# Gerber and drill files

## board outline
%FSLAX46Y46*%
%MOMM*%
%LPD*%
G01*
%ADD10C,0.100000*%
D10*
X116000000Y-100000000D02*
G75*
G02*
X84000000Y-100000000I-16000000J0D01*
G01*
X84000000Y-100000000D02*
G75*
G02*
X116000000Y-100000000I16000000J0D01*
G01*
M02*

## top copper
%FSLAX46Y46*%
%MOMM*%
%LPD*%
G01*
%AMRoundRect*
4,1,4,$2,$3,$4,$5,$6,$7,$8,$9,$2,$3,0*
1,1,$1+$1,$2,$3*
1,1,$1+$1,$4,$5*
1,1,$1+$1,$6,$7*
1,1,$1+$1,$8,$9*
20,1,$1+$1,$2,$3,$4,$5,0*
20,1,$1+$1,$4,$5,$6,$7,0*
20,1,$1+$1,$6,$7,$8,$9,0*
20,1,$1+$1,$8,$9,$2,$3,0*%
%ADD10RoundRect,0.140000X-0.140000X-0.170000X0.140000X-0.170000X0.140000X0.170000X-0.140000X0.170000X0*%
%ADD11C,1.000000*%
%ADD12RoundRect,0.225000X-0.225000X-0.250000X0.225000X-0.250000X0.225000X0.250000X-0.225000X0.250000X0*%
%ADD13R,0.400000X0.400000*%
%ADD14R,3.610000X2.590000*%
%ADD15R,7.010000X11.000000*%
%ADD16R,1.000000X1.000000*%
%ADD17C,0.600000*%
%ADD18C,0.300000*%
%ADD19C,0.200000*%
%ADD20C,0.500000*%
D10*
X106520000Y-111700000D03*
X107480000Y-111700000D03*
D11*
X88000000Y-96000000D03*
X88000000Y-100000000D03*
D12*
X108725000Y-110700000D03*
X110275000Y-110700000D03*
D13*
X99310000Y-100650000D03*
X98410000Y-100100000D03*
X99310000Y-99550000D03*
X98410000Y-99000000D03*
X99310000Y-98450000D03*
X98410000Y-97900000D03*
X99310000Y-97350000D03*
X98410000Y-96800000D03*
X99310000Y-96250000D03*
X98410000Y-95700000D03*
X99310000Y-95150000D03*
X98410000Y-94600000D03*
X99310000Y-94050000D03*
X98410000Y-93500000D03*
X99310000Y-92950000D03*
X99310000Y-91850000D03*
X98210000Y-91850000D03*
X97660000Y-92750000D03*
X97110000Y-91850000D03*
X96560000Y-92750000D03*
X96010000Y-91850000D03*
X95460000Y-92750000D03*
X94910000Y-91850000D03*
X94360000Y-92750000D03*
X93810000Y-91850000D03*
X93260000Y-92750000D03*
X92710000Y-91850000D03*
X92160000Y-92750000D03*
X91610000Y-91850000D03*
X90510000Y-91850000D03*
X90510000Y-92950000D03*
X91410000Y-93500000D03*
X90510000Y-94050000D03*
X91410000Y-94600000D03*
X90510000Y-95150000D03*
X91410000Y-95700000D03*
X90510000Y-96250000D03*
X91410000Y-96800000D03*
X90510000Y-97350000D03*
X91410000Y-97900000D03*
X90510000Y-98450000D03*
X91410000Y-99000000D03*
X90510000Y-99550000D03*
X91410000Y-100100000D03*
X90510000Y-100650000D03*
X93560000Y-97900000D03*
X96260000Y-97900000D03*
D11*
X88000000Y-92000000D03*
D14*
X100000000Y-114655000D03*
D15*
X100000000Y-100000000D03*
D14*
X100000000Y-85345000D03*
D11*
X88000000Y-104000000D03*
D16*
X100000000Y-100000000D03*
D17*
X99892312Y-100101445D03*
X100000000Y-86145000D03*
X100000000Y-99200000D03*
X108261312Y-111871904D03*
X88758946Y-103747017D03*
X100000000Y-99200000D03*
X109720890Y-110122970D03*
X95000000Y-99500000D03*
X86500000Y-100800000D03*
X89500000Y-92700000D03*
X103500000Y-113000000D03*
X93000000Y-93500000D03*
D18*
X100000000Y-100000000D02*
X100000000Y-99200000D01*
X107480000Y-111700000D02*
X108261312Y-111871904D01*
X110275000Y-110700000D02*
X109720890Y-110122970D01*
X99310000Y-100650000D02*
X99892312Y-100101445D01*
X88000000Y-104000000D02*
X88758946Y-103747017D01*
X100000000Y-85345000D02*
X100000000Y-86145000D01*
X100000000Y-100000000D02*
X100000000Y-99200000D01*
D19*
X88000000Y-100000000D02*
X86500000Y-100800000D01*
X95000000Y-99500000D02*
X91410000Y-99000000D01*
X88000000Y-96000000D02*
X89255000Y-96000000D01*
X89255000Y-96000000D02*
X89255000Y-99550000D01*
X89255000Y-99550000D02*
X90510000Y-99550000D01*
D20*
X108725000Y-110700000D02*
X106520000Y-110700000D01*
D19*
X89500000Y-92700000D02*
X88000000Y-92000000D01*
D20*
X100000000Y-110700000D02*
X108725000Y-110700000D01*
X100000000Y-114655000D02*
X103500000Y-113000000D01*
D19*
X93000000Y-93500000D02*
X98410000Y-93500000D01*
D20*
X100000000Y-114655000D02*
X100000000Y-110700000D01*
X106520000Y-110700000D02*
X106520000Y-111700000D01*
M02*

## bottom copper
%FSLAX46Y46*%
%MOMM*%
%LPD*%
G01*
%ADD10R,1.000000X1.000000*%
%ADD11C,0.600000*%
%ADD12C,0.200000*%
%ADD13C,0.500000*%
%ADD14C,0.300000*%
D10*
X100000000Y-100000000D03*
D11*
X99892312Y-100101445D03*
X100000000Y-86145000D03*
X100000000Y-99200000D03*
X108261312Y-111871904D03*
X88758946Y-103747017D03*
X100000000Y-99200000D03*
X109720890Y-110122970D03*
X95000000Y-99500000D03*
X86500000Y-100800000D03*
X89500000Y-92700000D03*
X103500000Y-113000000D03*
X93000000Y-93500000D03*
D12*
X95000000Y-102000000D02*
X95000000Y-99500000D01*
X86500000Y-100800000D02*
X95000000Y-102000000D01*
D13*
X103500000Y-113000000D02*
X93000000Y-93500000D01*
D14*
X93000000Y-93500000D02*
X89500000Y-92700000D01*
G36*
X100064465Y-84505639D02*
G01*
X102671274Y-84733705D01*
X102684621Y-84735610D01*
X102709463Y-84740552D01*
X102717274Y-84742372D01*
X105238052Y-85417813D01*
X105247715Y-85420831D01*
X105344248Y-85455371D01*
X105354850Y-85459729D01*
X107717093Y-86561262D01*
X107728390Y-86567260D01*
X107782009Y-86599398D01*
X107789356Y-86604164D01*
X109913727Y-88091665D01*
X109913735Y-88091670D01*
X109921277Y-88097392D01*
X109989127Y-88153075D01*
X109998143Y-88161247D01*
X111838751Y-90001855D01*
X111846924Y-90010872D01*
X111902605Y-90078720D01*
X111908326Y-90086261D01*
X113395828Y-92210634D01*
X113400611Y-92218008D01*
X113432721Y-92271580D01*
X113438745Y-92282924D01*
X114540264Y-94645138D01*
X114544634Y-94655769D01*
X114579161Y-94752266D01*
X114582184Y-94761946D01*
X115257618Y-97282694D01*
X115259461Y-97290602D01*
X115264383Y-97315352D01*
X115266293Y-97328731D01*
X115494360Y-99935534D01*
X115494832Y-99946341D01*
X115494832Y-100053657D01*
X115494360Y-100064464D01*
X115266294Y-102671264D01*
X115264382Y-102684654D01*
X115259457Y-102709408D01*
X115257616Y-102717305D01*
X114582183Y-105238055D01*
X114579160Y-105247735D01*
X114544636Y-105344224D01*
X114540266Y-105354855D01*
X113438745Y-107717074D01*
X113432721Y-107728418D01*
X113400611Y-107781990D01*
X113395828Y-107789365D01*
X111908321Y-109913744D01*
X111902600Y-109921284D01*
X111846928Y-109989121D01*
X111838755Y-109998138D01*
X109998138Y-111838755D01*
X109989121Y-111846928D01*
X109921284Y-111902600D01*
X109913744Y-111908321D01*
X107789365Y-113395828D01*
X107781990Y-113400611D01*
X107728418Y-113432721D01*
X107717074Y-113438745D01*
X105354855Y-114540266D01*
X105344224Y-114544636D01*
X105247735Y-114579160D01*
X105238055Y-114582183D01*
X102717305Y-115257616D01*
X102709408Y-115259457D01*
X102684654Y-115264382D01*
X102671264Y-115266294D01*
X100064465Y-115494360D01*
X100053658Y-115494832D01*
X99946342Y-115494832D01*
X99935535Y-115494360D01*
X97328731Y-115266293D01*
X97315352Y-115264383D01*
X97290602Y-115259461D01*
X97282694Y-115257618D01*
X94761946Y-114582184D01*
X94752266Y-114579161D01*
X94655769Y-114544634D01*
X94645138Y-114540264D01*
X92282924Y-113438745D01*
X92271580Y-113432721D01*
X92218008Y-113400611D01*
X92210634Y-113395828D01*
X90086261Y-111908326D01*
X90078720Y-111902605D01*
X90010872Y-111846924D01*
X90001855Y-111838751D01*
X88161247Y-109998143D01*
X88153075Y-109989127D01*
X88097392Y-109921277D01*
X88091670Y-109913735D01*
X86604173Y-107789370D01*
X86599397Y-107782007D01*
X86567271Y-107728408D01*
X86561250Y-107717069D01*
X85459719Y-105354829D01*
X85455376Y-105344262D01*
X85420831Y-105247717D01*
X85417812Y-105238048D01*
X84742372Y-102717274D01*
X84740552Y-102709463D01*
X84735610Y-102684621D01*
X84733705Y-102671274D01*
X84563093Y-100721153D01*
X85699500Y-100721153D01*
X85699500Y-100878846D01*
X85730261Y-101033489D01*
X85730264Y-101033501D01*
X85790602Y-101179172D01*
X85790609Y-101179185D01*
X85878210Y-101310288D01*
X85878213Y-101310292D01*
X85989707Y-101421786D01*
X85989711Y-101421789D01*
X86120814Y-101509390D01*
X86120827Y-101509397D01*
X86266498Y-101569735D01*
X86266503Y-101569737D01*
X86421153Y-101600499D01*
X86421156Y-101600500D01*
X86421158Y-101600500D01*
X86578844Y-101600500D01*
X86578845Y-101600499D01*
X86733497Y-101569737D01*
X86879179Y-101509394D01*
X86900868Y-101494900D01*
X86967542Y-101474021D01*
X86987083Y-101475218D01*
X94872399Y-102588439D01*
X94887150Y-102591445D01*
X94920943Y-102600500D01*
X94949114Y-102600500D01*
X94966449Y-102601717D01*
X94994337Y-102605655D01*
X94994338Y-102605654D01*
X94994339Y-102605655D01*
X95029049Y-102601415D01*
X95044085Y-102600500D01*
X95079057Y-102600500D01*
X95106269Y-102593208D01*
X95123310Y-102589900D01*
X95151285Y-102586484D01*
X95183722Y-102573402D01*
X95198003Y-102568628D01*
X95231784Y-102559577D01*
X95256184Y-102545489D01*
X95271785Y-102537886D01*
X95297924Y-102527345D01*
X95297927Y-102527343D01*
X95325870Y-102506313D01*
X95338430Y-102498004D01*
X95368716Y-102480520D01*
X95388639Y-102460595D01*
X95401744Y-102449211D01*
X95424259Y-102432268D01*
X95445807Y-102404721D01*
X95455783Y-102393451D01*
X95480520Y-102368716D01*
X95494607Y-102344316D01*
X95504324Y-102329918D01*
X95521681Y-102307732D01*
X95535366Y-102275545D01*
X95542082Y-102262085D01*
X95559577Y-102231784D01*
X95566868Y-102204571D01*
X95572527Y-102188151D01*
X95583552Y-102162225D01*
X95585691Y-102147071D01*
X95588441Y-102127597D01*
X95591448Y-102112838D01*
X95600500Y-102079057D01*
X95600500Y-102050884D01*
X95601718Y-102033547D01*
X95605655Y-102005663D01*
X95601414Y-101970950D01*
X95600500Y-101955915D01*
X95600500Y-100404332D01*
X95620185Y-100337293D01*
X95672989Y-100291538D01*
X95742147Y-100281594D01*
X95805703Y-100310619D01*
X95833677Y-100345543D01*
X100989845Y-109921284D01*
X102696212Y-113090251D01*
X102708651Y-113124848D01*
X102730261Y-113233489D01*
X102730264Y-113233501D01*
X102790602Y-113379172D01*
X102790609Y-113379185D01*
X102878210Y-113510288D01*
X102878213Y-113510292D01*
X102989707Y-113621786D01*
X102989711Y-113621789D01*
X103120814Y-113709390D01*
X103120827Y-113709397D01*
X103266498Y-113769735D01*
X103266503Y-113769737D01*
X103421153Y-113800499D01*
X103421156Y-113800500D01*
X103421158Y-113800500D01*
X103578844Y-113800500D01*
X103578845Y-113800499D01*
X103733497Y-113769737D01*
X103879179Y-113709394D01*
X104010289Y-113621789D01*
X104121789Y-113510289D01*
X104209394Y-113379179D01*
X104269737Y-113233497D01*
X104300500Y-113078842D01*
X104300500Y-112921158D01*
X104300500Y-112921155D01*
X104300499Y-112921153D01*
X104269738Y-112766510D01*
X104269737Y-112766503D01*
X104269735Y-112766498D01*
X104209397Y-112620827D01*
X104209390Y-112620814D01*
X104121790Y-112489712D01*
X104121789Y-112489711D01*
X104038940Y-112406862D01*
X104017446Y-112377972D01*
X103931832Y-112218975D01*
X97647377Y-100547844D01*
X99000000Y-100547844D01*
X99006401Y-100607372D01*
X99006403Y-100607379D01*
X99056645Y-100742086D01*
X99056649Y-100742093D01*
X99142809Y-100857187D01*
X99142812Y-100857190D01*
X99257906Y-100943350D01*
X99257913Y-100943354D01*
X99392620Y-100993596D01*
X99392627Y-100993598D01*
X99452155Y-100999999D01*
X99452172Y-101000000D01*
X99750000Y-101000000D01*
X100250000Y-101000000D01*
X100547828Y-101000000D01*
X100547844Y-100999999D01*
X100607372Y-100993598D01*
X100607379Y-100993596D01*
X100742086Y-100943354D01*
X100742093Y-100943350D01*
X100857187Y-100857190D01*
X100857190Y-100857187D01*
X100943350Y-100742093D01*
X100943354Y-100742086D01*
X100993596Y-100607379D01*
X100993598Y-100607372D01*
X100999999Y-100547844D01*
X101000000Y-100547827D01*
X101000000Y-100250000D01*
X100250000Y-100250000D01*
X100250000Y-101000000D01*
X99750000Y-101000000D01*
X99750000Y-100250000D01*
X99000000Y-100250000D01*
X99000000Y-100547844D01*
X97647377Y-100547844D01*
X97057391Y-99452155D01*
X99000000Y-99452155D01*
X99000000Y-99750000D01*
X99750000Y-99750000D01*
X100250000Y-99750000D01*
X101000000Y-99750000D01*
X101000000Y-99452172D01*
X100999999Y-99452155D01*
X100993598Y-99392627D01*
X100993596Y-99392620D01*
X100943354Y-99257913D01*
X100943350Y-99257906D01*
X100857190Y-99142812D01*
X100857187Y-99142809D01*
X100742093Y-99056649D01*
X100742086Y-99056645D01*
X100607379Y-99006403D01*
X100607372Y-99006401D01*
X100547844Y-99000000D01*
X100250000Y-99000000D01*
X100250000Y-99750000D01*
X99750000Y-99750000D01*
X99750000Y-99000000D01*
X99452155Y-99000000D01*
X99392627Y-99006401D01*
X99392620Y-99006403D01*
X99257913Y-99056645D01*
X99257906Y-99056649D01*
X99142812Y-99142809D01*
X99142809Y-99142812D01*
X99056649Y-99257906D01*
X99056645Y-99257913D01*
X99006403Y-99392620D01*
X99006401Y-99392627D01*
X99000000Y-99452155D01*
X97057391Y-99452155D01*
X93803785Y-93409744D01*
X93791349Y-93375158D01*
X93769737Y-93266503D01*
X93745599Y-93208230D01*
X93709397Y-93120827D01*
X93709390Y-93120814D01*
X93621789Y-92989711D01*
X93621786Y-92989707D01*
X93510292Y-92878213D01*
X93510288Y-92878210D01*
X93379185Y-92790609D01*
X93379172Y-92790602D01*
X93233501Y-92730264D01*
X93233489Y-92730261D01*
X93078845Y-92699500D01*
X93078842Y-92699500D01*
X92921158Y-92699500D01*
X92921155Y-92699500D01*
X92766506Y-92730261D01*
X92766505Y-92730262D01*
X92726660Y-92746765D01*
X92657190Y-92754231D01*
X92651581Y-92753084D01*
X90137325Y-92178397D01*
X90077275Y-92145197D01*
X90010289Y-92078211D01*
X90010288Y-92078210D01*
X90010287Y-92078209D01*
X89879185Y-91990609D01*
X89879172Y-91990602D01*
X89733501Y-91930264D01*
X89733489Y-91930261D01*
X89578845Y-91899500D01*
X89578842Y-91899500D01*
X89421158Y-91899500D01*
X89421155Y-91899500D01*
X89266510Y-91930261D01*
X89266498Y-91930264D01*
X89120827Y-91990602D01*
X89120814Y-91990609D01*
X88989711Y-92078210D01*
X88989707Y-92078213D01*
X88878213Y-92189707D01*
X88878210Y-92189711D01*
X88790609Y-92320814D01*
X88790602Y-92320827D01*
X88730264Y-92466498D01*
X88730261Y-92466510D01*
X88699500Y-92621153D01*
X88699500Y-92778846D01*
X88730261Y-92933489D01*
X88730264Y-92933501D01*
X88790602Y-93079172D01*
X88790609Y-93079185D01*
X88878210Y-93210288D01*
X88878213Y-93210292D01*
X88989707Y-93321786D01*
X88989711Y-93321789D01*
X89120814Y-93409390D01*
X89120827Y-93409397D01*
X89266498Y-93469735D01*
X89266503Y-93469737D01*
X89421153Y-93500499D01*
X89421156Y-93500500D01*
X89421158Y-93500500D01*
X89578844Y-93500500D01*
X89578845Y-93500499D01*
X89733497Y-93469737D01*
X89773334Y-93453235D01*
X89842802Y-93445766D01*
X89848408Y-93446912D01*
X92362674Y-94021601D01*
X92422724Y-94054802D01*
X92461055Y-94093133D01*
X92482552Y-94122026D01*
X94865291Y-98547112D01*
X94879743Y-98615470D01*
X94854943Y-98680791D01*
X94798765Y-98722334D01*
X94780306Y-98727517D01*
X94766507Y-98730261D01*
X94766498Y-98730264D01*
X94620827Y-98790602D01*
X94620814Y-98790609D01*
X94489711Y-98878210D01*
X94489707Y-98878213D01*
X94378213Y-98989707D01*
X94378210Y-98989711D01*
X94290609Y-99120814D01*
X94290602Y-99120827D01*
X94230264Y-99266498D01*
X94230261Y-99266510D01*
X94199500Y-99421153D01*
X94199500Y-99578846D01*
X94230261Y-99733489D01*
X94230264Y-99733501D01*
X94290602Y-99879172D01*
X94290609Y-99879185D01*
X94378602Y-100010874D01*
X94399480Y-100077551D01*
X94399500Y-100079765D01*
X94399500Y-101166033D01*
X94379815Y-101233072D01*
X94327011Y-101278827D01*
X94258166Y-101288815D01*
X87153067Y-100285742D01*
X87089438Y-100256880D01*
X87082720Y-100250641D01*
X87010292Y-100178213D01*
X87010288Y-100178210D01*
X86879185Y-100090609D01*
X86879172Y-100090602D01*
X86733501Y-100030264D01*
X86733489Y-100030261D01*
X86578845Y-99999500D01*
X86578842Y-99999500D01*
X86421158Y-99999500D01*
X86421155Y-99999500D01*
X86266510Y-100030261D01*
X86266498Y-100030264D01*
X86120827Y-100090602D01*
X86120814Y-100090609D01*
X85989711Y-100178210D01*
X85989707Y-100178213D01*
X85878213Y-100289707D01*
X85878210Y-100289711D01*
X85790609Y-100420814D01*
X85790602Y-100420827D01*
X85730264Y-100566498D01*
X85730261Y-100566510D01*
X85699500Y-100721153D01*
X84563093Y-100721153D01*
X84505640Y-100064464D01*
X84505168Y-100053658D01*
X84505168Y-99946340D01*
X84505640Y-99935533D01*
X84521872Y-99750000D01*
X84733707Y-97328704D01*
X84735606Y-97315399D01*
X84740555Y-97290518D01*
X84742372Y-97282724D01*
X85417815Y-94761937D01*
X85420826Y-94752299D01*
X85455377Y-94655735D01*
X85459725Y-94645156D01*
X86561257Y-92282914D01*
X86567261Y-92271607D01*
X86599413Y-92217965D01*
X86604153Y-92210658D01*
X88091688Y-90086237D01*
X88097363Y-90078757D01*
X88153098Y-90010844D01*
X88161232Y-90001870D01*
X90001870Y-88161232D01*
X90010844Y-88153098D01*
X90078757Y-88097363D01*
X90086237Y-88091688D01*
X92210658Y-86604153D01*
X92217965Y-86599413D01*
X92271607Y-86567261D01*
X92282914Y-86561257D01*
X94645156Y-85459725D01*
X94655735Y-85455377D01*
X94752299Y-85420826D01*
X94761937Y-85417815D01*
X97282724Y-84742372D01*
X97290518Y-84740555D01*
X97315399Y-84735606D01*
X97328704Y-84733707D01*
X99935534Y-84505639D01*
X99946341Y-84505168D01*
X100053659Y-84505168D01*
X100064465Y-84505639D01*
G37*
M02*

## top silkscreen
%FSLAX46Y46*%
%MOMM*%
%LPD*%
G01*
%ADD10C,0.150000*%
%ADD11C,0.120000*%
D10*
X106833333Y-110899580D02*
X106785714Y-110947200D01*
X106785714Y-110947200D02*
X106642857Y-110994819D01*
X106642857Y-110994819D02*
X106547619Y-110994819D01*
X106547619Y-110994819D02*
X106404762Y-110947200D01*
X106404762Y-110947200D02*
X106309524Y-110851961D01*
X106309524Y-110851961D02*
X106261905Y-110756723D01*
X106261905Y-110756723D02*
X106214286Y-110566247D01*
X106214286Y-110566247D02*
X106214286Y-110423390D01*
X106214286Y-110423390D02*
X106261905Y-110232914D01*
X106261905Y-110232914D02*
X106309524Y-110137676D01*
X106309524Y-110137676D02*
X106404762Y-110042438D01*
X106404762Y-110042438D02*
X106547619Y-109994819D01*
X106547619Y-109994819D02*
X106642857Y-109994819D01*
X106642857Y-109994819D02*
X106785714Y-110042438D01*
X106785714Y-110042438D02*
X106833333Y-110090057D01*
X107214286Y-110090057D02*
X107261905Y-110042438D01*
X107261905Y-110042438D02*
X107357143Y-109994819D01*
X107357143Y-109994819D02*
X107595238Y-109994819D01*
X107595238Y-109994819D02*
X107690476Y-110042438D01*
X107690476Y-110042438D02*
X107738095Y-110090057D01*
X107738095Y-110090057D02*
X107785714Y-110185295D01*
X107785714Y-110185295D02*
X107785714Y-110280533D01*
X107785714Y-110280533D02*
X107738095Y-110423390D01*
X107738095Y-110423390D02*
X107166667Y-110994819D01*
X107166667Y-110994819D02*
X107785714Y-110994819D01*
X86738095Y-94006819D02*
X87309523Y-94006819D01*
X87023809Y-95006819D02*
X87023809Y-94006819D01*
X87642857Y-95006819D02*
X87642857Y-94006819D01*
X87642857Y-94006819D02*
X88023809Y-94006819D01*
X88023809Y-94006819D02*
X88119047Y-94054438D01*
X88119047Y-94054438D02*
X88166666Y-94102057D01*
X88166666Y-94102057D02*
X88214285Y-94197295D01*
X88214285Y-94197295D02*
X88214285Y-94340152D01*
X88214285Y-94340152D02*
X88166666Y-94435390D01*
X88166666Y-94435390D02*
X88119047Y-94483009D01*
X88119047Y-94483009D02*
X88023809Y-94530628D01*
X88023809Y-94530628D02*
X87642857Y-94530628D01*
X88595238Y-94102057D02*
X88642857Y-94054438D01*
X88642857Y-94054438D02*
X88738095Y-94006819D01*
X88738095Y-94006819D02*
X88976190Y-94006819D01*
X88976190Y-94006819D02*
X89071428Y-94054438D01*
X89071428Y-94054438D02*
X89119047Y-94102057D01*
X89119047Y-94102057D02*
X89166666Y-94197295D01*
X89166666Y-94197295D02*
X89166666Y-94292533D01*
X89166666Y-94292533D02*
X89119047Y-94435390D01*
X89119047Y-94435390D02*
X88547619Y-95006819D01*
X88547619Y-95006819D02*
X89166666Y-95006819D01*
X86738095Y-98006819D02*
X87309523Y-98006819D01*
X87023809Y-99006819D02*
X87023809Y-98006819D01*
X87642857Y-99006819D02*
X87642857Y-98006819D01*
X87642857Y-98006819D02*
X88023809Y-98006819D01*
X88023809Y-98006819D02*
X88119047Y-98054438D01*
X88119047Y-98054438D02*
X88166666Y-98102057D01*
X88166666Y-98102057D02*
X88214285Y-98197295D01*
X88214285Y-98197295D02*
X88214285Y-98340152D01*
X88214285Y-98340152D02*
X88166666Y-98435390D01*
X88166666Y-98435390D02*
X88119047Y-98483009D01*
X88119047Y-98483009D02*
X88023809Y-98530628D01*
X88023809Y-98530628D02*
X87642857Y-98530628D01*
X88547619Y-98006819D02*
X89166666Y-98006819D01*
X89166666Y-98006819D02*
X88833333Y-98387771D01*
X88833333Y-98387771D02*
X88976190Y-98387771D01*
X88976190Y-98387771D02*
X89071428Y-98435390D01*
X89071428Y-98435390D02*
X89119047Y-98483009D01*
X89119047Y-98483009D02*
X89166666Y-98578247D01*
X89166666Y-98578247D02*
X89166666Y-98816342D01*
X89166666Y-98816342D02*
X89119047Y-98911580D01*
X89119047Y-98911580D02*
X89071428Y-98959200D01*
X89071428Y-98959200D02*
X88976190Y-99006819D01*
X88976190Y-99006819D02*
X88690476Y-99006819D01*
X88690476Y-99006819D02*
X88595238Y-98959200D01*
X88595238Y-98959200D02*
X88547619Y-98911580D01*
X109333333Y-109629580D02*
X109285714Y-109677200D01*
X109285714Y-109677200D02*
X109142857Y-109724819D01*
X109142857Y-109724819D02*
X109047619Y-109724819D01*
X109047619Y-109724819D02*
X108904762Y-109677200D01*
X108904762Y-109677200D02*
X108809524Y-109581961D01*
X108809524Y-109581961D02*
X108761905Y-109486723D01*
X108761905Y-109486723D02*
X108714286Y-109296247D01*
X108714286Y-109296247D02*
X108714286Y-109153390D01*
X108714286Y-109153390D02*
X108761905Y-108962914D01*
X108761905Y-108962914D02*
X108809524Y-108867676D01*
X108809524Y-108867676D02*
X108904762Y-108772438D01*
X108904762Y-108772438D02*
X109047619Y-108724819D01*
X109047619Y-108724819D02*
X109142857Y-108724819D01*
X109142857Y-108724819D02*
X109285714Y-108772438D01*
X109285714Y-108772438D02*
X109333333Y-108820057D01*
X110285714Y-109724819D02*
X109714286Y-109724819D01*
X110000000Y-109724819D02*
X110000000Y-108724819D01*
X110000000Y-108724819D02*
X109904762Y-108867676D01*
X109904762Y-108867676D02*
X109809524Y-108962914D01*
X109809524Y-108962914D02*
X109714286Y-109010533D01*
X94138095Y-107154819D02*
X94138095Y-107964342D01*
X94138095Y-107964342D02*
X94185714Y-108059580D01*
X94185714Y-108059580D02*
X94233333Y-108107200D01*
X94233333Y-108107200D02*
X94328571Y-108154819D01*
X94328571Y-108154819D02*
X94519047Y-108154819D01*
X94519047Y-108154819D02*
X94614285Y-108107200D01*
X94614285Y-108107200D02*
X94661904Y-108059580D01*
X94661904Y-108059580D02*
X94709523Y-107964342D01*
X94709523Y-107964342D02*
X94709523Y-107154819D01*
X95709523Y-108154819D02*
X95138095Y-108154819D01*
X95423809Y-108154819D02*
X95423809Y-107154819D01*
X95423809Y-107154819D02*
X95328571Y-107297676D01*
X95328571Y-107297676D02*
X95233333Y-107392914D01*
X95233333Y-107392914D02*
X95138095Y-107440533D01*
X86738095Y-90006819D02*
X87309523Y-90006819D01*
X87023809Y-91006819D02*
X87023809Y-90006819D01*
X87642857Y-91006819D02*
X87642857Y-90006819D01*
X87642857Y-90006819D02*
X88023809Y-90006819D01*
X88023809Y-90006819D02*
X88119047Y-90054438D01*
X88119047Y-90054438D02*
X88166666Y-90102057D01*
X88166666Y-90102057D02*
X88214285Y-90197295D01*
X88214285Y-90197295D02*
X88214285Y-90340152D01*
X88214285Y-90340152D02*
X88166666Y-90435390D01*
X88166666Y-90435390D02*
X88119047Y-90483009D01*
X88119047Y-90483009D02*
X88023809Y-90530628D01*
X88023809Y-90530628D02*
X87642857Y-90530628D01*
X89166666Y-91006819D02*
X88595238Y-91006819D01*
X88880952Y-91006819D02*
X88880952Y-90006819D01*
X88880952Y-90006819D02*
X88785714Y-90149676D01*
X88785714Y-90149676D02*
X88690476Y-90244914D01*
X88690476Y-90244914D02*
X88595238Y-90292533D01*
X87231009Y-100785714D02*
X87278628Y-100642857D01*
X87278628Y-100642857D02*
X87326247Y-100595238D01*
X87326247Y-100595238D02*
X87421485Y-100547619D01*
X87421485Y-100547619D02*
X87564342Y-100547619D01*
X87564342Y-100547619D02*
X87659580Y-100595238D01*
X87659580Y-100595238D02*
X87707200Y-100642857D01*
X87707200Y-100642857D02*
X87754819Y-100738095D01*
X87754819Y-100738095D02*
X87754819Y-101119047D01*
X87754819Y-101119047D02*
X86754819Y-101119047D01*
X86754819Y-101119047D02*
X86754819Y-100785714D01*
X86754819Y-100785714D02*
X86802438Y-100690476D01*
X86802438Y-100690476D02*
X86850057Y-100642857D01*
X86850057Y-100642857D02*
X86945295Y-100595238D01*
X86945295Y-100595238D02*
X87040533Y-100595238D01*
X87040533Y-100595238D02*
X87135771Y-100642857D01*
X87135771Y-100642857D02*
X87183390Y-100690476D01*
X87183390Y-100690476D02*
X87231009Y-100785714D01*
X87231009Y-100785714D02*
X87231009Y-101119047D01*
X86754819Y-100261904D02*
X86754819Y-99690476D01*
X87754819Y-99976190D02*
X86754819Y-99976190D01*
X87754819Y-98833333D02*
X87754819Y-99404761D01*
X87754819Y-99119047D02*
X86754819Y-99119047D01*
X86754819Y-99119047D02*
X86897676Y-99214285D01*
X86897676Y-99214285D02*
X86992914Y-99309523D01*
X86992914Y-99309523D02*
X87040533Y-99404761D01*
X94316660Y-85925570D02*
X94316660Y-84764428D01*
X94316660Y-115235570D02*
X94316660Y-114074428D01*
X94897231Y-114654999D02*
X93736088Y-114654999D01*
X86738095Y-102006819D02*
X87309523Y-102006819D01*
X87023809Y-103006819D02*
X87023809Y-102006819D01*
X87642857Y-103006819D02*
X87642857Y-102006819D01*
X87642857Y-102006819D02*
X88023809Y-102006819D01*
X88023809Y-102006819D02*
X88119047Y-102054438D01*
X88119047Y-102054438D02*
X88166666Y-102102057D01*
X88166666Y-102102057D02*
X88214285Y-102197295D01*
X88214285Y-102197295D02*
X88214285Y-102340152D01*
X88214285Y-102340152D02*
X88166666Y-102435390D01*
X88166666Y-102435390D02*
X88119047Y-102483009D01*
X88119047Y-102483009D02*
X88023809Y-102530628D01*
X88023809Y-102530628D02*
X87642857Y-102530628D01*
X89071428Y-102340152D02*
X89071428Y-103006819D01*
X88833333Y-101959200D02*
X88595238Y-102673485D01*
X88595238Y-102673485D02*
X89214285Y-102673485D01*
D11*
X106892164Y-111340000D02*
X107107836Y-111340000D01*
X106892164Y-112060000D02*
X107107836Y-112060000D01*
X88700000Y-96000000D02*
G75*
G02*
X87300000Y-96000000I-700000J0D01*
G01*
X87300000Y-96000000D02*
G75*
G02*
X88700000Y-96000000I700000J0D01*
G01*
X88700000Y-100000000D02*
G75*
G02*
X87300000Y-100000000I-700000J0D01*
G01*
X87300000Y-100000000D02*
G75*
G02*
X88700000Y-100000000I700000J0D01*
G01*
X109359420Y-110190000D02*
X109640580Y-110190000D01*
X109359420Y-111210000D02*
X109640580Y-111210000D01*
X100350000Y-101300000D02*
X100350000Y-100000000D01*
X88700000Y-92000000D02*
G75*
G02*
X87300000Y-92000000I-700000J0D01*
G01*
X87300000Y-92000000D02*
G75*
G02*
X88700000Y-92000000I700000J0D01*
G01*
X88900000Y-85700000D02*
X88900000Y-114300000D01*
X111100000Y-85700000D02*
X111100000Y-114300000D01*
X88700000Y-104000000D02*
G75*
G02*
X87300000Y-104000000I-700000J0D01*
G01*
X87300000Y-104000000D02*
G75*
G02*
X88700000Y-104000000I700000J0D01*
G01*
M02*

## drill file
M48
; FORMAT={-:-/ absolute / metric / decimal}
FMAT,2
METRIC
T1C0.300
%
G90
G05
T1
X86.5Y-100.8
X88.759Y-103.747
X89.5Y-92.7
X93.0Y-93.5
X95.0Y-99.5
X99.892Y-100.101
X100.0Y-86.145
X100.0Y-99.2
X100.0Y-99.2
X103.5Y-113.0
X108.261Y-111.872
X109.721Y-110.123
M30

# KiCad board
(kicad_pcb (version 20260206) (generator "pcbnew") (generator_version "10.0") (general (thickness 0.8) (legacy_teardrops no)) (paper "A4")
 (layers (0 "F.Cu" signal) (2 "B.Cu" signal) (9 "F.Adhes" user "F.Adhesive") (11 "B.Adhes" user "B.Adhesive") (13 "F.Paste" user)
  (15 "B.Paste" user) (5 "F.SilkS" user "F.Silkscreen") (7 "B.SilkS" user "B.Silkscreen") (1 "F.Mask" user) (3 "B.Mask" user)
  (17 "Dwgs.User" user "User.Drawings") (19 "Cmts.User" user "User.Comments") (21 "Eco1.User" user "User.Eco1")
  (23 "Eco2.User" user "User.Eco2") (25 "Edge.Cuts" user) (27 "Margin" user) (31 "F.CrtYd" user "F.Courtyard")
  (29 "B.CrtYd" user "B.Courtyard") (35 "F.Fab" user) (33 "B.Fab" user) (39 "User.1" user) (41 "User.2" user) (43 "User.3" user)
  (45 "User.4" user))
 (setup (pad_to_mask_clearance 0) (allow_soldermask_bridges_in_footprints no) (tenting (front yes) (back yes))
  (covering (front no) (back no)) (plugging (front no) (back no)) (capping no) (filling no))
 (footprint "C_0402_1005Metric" (layer "F.Cu") (at 107 111.7)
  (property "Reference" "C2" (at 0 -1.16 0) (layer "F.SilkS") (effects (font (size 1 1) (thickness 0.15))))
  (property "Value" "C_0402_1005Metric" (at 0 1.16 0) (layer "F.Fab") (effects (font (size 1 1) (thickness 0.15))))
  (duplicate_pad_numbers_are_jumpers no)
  (fp_line (start -0.107836 -0.36) (end 0.107836 -0.36) (stroke (width 0.12) (type solid)) (layer "F.SilkS"))
  (fp_line (start -0.107836 0.36) (end 0.107836 0.36) (stroke (width 0.12) (type solid)) (layer "F.SilkS"))
  (pad "1" smd roundrect (at -0.48 0) (size 0.56 0.62) (layers "F.Cu" "F.Mask" "F.Paste") (roundrect_rratio 0.25) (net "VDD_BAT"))
  (pad "2" smd roundrect (at 0.48 0) (size 0.56 0.62) (layers "F.Cu" "F.Mask" "F.Paste") (roundrect_rratio 0.25) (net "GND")))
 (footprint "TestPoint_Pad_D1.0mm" (layer "F.Cu") (at 88 96)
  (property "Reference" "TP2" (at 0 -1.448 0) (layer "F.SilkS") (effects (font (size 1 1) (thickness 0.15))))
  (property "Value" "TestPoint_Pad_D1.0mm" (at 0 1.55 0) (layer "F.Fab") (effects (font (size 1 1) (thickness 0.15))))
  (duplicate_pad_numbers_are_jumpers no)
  (fp_circle (center 0 0) (end 0 0.7) (stroke (width 0.12) (type solid)) (fill no) (layer "F.SilkS"))
  (pad "1" smd circle (at 0 0) (size 1 1) (layers "F.Cu" "F.Mask") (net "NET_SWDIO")))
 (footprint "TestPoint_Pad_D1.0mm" (layer "F.Cu") (at 88 100)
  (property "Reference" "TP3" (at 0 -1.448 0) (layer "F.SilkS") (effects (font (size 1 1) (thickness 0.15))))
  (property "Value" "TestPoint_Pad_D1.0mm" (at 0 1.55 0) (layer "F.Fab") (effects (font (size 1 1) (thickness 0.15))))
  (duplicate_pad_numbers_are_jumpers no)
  (fp_circle (center 0 0) (end 0 0.7) (stroke (width 0.12) (type solid)) (fill no) (layer "F.SilkS"))
  (pad "1" smd circle (at 0 0) (size 1 1) (layers "F.Cu" "F.Mask") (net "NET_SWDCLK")))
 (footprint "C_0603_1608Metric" (layer "F.Cu") (at 109.5 110.7)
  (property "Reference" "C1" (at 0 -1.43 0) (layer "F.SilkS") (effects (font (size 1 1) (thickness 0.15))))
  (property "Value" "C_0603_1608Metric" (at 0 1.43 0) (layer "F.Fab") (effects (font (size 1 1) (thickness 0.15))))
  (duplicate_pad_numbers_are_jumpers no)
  (fp_line (start -0.14058 -0.51) (end 0.14058 -0.51) (stroke (width 0.12) (type solid)) (layer "F.SilkS"))
  (fp_line (start -0.14058 0.51) (end 0.14058 0.51) (stroke (width 0.12) (type solid)) (layer "F.SilkS"))
  (pad "1" smd roundrect (at -0.775 0) (size 0.9 0.95) (layers "F.Cu" "F.Mask" "F.Paste") (roundrect_rratio 0.25) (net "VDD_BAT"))
  (pad "2" smd roundrect (at 0.775 0) (size 0.9 0.95) (layers "F.Cu" "F.Mask" "F.Paste") (roundrect_rratio 0.25) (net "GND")))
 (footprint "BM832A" (layer "F.Cu") (at 100 106.2 180)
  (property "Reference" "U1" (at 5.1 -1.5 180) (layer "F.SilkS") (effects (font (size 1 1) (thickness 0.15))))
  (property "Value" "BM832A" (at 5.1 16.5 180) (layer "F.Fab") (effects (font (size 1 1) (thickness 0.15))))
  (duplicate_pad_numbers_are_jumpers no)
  (fp_line (start -0.35 4.9) (end -0.35 6.2) (stroke (width 0.12) (type solid)) (layer "F.SilkS"))
  (pad "1" smd rect (at 0.69 5.55 180) (size 0.4 0.4) (layers "F.Cu" "F.Mask" "F.Paste") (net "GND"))
  (pad "2" smd rect (at 1.59 6.1 180) (size 0.4 0.4) (layers "F.Cu" "F.Mask" "F.Paste"))
  (pad "3" smd rect (at 0.69 6.65 180) (size 0.4 0.4) (layers "F.Cu" "F.Mask" "F.Paste"))
  (pad "4" smd rect (at 1.59 7.2 180) (size 0.4 0.4) (layers "F.Cu" "F.Mask" "F.Paste"))
  (pad "5" smd rect (at 0.69 7.75 180) (size 0.4 0.4) (layers "F.Cu" "F.Mask" "F.Paste"))
  (pad "6" smd rect (at 1.59 8.3 180) (size 0.4 0.4) (layers "F.Cu" "F.Mask" "F.Paste"))
  (pad "7" smd rect (at 0.69 8.85 180) (size 0.4 0.4) (layers "F.Cu" "F.Mask" "F.Paste"))
  (pad "8" smd rect (at 1.59 9.4 180) (size 0.4 0.4) (layers "F.Cu" "F.Mask" "F.Paste"))
  (pad "9" smd rect (at 0.69 9.95 180) (size 0.4 0.4) (layers "F.Cu" "F.Mask" "F.Paste"))
  (pad "10" smd rect (at 1.59 10.5 180) (size 0.4 0.4) (layers "F.Cu" "F.Mask" "F.Paste"))
  (pad "11" smd rect (at 0.69 11.05 180) (size 0.4 0.4) (layers "F.Cu" "F.Mask" "F.Paste"))
  (pad "12" smd rect (at 1.59 11.6 180) (size 0.4 0.4) (layers "F.Cu" "F.Mask" "F.Paste"))
  (pad "13" smd rect (at 0.69 12.15 180) (size 0.4 0.4) (layers "F.Cu" "F.Mask" "F.Paste"))
  (pad "14" smd rect (at 1.59 12.7 180) (size 0.4 0.4) (layers "F.Cu" "F.Mask" "F.Paste") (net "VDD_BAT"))
  (pad "15" smd rect (at 0.69 13.25 180) (size 0.4 0.4) (layers "F.Cu" "F.Mask" "F.Paste"))
  (pad "16" smd rect (at 0.69 14.35 180) (size 0.4 0.4) (layers "F.Cu" "F.Mask" "F.Paste"))
  (pad "17" smd rect (at 1.79 14.35 180) (size 0.4 0.4) (layers "F.Cu" "F.Mask" "F.Paste"))
  (pad "18" smd rect (at 2.34 13.45 180) (size 0.4 0.4) (layers "F.Cu" "F.Mask" "F.Paste"))
  (pad "19" smd rect (at 2.89 14.35 180) (size 0.4 0.4) (layers "F.Cu" "F.Mask" "F.Paste"))
  (pad "20" smd rect (at 3.44 13.45 180) (size 0.4 0.4) (layers "F.Cu" "F.Mask" "F.Paste"))
  (pad "21" smd rect (at 3.99 14.35 180) (size 0.4 0.4) (layers "F.Cu" "F.Mask" "F.Paste"))
  (pad "22" smd rect (at 4.54 13.45 180) (size 0.4 0.4) (layers "F.Cu" "F.Mask" "F.Paste"))
  (pad "23" smd rect (at 5.09 14.35 180) (size 0.4 0.4) (layers "F.Cu" "F.Mask" "F.Paste"))
  (pad "24" smd rect (at 5.64 13.45 180) (size 0.4 0.4) (layers "F.Cu" "F.Mask" "F.Paste"))
  (pad "25" smd rect (at 6.19 14.35 180) (size 0.4 0.4) (layers "F.Cu" "F.Mask" "F.Paste"))
  (pad "26" smd rect (at 6.74 13.45 180) (size 0.4 0.4) (layers "F.Cu" "F.Mask" "F.Paste"))
  (pad "27" smd rect (at 7.29 14.35 180) (size 0.4 0.4) (layers "F.Cu" "F.Mask" "F.Paste"))
  (pad "28" smd rect (at 7.84 13.45 180) (size 0.4 0.4) (layers "F.Cu" "F.Mask" "F.Paste"))
  (pad "29" smd rect (at 8.39 14.35 180) (size 0.4 0.4) (layers "F.Cu" "F.Mask" "F.Paste"))
  (pad "30" smd rect (at 9.49 14.35 180) (size 0.4 0.4) (layers "F.Cu" "F.Mask" "F.Paste"))
  (pad "31" smd rect (at 9.49 13.25 180) (size 0.4 0.4) (layers "F.Cu" "F.Mask" "F.Paste"))
  (pad "32" smd rect (at 8.59 12.7 180) (size 0.4 0.4) (layers "F.Cu" "F.Mask" "F.Paste"))
  (pad "33" smd rect (at 9.49 12.15 180) (size 0.4 0.4) (layers "F.Cu" "F.Mask" "F.Paste"))
  (pad "34" smd rect (at 8.59 11.6 180) (size 0.4 0.4) (layers "F.Cu" "F.Mask" "F.Paste"))
  (pad "35" smd rect (at 9.49 11.05 180) (size 0.4 0.4) (layers "F.Cu" "F.Mask" "F.Paste"))
  (pad "36" smd rect (at 8.59 10.5 180) (size 0.4 0.4) (layers "F.Cu" "F.Mask" "F.Paste"))
  (pad "37" smd rect (at 9.49 9.95 180) (size 0.4 0.4) (layers "F.Cu" "F.Mask" "F.Paste"))
  (pad "38" smd rect (at 8.59 9.4 180) (size 0.4 0.4) (layers "F.Cu" "F.Mask" "F.Paste"))
  (pad "39" smd rect (at 9.49 8.85 180) (size 0.4 0.4) (layers "F.Cu" "F.Mask" "F.Paste"))
  (pad "40" smd rect (at 8.59 8.3 180) (size 0.4 0.4) (layers "F.Cu" "F.Mask" "F.Paste"))
  (pad "41" smd rect (at 9.49 7.75 180) (size 0.4 0.4) (layers "F.Cu" "F.Mask" "F.Paste"))
  (pad "42" smd rect (at 8.59 7.2 180) (size 0.4 0.4) (layers "F.Cu" "F.Mask" "F.Paste") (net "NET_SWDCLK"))
  (pad "43" smd rect (at 9.49 6.65 180) (size 0.4 0.4) (layers "F.Cu" "F.Mask" "F.Paste") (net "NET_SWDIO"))
  (pad "44" smd rect (at 8.59 6.1 180) (size 0.4 0.4) (layers "F.Cu" "F.Mask" "F.Paste"))
  (pad "45" smd rect (at 9.49 5.55 180) (size 0.4 0.4) (layers "F.Cu" "F.Mask" "F.Paste"))
  (pad "46" smd rect (at 6.44 8.3 180) (size 0.4 0.4) (layers "F.Cu" "F.Mask" "F.Paste"))
  (pad "47" smd rect (at 3.74 8.3 180) (size 0.4 0.4) (layers "F.Cu" "F.Mask" "F.Paste")))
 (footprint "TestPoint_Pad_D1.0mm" (layer "F.Cu") (at 88 92)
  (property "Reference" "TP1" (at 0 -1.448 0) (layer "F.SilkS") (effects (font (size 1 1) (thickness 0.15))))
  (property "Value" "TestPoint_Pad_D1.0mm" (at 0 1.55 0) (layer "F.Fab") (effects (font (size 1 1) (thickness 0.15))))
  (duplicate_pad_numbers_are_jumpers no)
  (fp_circle (center 0 0) (end 0 0.7) (stroke (width 0.12) (type solid)) (fill no) (layer "F.SilkS"))
  (pad "1" smd circle (at 0 0) (size 1 1) (layers "F.Cu" "F.Mask") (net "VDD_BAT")))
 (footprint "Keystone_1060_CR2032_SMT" (layer "F.Cu") (at 100 100 -90)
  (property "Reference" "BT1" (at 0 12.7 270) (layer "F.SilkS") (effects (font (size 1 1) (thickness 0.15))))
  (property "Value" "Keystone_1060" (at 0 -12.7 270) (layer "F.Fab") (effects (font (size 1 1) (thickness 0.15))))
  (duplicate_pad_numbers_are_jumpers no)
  (fp_line (start -14.3 11.1) (end 14.3 11.1) (stroke (width 0.12) (type solid)) (layer "F.SilkS"))
  (fp_line (start -14.3 -11.1) (end 14.3 -11.1) (stroke (width 0.12) (type solid)) (layer "F.SilkS"))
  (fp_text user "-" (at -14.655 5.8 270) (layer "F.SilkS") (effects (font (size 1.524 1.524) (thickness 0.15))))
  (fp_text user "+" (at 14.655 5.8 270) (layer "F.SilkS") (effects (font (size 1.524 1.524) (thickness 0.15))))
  (pad "1" smd rect (at 14.655 0 270) (size 2.59 3.61) (layers "F.Cu" "F.Mask" "F.Paste") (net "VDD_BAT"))
  (pad "2" smd rect (at 0 0 270) (size 11 7.01) (layers "F.Cu" "F.Mask" "F.Paste") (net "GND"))
  (pad "3" smd rect (at -14.655 0 270) (size 2.59 3.61) (layers "F.Cu" "F.Mask" "F.Paste") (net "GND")))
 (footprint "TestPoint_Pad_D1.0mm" (layer "F.Cu") (at 88 104)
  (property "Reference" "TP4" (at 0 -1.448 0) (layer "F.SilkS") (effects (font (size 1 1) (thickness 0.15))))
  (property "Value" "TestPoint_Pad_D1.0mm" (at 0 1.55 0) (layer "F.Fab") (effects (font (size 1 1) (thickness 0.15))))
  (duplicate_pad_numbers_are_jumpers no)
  (fp_circle (center 0 0) (end 0 0.7) (stroke (width 0.12) (type solid)) (fill no) (layer "F.SilkS"))
  (pad "1" smd circle (at 0 0) (size 1 1) (layers "F.Cu" "F.Mask") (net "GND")))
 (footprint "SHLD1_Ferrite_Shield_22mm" (layer "B.Cu") (at 100 100 180)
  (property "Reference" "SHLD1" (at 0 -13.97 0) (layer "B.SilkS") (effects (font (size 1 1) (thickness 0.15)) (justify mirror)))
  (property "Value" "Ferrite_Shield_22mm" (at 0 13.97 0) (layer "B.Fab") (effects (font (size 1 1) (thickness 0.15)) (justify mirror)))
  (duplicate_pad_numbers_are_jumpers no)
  (pad "1" smd rect (at 0 0 180) (size 1 1) (layers "*.Cu" "*.Paste" "*.Mask") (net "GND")))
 (gr_circle (center 100 100) (end 116 100) (stroke (width 0.1) (type default)) (fill no) (layer "Edge.Cuts"))
 (segment (start 100 100) (end 100 99.2) (width 0.3) (layer "F.Cu") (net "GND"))
 (segment (start 107.48 111.7) (end 108.261312 111.871904) (width 0.3) (layer "F.Cu") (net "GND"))
 (segment (start 110.275 110.7) (end 109.72089 110.12297) (width 0.3) (layer "F.Cu") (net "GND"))
 (segment (start 99.31 100.65) (end 99.892312 100.101445) (width 0.3) (layer "F.Cu") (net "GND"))
 (segment (start 88 104) (end 88.758946 103.747017) (width 0.3) (layer "F.Cu") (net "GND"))
 (segment (start 100 85.345) (end 100 86.145) (width 0.3) (layer "F.Cu") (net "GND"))
 (segment (start 100 100) (end 100 99.2) (width 0.3) (layer "F.Cu") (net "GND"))
 (via (at 99.892312 100.101445) (size 0.6) (drill 0.3) (layers "F.Cu" "B.Cu") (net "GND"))
 (via (at 100 86.145) (size 0.6) (drill 0.3) (layers "F.Cu" "B.Cu") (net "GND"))
 (via (at 100 99.2) (size 0.6) (drill 0.3) (layers "F.Cu" "B.Cu") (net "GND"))
 (via (at 108.261312 111.871904) (size 0.6) (drill 0.3) (layers "F.Cu" "B.Cu") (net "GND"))
 (via (at 88.758946 103.747017) (size 0.6) (drill 0.3) (layers "F.Cu" "B.Cu") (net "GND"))
 (via (at 100 99.2) (size 0.6) (drill 0.3) (layers "F.Cu" "B.Cu") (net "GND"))
 (via (at 109.72089 110.12297) (size 0.6) (drill 0.3) (layers "F.Cu" "B.Cu") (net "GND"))
 (segment (start 88 100) (end 86.5 100.8) (width 0.2) (layer "F.Cu") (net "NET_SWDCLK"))
 (segment (start 95 99.5) (end 91.41 99) (width 0.2) (layer "F.Cu") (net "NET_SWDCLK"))
 (via (at 95 99.5) (size 0.6) (drill 0.3) (layers "F.Cu" "B.Cu") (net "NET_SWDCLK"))
 (via (at 86.5 100.8) (size 0.6) (drill 0.3) (layers "F.Cu" "B.Cu") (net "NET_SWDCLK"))
 (segment (start 95 102) (end 95 99.5) (width 0.2) (layer "B.Cu") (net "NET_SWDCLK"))
 (segment (start 86.5 100.8) (end 95 102) (width 0.2) (layer "B.Cu") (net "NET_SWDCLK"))
 (segment (start 88 96) (end 89.255 96) (width 0.2) (layer "F.Cu") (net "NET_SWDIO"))
 (segment (start 89.255 96) (end 89.255 99.55) (width 0.2) (layer "F.Cu") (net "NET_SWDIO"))
 (segment (start 89.255 99.55) (end 90.51 99.55) (width 0.2) (layer "F.Cu") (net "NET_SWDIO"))
 (segment (start 108.725 110.7) (end 106.52 110.7) (width 0.5) (layer "F.Cu") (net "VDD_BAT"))
 (segment (start 89.5 92.7) (end 88 92) (width 0.2) (layer "F.Cu") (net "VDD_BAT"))
 (segment (start 100 110.7) (end 108.725 110.7) (width 0.5) (layer "F.Cu") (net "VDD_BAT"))
 (segment (start 100 114.655) (end 103.5 113) (width 0.5) (layer "F.Cu") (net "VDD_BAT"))
 (segment (start 93 93.5) (end 98.41 93.5) (width 0.2) (layer "F.Cu") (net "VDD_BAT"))
 (segment (start 100 114.655) (end 100 110.7) (width 0.5) (layer "F.Cu") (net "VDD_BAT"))
 (segment (start 106.52 110.7) (end 106.52 111.7) (width 0.5) (layer "F.Cu") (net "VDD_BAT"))
 (via (at 89.5 92.7) (size 0.6) (drill 0.3) (layers "F.Cu" "B.Cu") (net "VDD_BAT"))
 (via (at 103.5 113) (size 0.6) (drill 0.3) (layers "F.Cu" "B.Cu") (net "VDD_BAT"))
 (via (at 93 93.5) (size 0.6) (drill 0.3) (layers "F.Cu" "B.Cu") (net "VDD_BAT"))
 (segment (start 103.5 113) (end 93 93.5) (width 0.5) (layer "B.Cu") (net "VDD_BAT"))
 (segment (start 93 93.5) (end 89.5 92.7) (width 0.3) (layer "B.Cu") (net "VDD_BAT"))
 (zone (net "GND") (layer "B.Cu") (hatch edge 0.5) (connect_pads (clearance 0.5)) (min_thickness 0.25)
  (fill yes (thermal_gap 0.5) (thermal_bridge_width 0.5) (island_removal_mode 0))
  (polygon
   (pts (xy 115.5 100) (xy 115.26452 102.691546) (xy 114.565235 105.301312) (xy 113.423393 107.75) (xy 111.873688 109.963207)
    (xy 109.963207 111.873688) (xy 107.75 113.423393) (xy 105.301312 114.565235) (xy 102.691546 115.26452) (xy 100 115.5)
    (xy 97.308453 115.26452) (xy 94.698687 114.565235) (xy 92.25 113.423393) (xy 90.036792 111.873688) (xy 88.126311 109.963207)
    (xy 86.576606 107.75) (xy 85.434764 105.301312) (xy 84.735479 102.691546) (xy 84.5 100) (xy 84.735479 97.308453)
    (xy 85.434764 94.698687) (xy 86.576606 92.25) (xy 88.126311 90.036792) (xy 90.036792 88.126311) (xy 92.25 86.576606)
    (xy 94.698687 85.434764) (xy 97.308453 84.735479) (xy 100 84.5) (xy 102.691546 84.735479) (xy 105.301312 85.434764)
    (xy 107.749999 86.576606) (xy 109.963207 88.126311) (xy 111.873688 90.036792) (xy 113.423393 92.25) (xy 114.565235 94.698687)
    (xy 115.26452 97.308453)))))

